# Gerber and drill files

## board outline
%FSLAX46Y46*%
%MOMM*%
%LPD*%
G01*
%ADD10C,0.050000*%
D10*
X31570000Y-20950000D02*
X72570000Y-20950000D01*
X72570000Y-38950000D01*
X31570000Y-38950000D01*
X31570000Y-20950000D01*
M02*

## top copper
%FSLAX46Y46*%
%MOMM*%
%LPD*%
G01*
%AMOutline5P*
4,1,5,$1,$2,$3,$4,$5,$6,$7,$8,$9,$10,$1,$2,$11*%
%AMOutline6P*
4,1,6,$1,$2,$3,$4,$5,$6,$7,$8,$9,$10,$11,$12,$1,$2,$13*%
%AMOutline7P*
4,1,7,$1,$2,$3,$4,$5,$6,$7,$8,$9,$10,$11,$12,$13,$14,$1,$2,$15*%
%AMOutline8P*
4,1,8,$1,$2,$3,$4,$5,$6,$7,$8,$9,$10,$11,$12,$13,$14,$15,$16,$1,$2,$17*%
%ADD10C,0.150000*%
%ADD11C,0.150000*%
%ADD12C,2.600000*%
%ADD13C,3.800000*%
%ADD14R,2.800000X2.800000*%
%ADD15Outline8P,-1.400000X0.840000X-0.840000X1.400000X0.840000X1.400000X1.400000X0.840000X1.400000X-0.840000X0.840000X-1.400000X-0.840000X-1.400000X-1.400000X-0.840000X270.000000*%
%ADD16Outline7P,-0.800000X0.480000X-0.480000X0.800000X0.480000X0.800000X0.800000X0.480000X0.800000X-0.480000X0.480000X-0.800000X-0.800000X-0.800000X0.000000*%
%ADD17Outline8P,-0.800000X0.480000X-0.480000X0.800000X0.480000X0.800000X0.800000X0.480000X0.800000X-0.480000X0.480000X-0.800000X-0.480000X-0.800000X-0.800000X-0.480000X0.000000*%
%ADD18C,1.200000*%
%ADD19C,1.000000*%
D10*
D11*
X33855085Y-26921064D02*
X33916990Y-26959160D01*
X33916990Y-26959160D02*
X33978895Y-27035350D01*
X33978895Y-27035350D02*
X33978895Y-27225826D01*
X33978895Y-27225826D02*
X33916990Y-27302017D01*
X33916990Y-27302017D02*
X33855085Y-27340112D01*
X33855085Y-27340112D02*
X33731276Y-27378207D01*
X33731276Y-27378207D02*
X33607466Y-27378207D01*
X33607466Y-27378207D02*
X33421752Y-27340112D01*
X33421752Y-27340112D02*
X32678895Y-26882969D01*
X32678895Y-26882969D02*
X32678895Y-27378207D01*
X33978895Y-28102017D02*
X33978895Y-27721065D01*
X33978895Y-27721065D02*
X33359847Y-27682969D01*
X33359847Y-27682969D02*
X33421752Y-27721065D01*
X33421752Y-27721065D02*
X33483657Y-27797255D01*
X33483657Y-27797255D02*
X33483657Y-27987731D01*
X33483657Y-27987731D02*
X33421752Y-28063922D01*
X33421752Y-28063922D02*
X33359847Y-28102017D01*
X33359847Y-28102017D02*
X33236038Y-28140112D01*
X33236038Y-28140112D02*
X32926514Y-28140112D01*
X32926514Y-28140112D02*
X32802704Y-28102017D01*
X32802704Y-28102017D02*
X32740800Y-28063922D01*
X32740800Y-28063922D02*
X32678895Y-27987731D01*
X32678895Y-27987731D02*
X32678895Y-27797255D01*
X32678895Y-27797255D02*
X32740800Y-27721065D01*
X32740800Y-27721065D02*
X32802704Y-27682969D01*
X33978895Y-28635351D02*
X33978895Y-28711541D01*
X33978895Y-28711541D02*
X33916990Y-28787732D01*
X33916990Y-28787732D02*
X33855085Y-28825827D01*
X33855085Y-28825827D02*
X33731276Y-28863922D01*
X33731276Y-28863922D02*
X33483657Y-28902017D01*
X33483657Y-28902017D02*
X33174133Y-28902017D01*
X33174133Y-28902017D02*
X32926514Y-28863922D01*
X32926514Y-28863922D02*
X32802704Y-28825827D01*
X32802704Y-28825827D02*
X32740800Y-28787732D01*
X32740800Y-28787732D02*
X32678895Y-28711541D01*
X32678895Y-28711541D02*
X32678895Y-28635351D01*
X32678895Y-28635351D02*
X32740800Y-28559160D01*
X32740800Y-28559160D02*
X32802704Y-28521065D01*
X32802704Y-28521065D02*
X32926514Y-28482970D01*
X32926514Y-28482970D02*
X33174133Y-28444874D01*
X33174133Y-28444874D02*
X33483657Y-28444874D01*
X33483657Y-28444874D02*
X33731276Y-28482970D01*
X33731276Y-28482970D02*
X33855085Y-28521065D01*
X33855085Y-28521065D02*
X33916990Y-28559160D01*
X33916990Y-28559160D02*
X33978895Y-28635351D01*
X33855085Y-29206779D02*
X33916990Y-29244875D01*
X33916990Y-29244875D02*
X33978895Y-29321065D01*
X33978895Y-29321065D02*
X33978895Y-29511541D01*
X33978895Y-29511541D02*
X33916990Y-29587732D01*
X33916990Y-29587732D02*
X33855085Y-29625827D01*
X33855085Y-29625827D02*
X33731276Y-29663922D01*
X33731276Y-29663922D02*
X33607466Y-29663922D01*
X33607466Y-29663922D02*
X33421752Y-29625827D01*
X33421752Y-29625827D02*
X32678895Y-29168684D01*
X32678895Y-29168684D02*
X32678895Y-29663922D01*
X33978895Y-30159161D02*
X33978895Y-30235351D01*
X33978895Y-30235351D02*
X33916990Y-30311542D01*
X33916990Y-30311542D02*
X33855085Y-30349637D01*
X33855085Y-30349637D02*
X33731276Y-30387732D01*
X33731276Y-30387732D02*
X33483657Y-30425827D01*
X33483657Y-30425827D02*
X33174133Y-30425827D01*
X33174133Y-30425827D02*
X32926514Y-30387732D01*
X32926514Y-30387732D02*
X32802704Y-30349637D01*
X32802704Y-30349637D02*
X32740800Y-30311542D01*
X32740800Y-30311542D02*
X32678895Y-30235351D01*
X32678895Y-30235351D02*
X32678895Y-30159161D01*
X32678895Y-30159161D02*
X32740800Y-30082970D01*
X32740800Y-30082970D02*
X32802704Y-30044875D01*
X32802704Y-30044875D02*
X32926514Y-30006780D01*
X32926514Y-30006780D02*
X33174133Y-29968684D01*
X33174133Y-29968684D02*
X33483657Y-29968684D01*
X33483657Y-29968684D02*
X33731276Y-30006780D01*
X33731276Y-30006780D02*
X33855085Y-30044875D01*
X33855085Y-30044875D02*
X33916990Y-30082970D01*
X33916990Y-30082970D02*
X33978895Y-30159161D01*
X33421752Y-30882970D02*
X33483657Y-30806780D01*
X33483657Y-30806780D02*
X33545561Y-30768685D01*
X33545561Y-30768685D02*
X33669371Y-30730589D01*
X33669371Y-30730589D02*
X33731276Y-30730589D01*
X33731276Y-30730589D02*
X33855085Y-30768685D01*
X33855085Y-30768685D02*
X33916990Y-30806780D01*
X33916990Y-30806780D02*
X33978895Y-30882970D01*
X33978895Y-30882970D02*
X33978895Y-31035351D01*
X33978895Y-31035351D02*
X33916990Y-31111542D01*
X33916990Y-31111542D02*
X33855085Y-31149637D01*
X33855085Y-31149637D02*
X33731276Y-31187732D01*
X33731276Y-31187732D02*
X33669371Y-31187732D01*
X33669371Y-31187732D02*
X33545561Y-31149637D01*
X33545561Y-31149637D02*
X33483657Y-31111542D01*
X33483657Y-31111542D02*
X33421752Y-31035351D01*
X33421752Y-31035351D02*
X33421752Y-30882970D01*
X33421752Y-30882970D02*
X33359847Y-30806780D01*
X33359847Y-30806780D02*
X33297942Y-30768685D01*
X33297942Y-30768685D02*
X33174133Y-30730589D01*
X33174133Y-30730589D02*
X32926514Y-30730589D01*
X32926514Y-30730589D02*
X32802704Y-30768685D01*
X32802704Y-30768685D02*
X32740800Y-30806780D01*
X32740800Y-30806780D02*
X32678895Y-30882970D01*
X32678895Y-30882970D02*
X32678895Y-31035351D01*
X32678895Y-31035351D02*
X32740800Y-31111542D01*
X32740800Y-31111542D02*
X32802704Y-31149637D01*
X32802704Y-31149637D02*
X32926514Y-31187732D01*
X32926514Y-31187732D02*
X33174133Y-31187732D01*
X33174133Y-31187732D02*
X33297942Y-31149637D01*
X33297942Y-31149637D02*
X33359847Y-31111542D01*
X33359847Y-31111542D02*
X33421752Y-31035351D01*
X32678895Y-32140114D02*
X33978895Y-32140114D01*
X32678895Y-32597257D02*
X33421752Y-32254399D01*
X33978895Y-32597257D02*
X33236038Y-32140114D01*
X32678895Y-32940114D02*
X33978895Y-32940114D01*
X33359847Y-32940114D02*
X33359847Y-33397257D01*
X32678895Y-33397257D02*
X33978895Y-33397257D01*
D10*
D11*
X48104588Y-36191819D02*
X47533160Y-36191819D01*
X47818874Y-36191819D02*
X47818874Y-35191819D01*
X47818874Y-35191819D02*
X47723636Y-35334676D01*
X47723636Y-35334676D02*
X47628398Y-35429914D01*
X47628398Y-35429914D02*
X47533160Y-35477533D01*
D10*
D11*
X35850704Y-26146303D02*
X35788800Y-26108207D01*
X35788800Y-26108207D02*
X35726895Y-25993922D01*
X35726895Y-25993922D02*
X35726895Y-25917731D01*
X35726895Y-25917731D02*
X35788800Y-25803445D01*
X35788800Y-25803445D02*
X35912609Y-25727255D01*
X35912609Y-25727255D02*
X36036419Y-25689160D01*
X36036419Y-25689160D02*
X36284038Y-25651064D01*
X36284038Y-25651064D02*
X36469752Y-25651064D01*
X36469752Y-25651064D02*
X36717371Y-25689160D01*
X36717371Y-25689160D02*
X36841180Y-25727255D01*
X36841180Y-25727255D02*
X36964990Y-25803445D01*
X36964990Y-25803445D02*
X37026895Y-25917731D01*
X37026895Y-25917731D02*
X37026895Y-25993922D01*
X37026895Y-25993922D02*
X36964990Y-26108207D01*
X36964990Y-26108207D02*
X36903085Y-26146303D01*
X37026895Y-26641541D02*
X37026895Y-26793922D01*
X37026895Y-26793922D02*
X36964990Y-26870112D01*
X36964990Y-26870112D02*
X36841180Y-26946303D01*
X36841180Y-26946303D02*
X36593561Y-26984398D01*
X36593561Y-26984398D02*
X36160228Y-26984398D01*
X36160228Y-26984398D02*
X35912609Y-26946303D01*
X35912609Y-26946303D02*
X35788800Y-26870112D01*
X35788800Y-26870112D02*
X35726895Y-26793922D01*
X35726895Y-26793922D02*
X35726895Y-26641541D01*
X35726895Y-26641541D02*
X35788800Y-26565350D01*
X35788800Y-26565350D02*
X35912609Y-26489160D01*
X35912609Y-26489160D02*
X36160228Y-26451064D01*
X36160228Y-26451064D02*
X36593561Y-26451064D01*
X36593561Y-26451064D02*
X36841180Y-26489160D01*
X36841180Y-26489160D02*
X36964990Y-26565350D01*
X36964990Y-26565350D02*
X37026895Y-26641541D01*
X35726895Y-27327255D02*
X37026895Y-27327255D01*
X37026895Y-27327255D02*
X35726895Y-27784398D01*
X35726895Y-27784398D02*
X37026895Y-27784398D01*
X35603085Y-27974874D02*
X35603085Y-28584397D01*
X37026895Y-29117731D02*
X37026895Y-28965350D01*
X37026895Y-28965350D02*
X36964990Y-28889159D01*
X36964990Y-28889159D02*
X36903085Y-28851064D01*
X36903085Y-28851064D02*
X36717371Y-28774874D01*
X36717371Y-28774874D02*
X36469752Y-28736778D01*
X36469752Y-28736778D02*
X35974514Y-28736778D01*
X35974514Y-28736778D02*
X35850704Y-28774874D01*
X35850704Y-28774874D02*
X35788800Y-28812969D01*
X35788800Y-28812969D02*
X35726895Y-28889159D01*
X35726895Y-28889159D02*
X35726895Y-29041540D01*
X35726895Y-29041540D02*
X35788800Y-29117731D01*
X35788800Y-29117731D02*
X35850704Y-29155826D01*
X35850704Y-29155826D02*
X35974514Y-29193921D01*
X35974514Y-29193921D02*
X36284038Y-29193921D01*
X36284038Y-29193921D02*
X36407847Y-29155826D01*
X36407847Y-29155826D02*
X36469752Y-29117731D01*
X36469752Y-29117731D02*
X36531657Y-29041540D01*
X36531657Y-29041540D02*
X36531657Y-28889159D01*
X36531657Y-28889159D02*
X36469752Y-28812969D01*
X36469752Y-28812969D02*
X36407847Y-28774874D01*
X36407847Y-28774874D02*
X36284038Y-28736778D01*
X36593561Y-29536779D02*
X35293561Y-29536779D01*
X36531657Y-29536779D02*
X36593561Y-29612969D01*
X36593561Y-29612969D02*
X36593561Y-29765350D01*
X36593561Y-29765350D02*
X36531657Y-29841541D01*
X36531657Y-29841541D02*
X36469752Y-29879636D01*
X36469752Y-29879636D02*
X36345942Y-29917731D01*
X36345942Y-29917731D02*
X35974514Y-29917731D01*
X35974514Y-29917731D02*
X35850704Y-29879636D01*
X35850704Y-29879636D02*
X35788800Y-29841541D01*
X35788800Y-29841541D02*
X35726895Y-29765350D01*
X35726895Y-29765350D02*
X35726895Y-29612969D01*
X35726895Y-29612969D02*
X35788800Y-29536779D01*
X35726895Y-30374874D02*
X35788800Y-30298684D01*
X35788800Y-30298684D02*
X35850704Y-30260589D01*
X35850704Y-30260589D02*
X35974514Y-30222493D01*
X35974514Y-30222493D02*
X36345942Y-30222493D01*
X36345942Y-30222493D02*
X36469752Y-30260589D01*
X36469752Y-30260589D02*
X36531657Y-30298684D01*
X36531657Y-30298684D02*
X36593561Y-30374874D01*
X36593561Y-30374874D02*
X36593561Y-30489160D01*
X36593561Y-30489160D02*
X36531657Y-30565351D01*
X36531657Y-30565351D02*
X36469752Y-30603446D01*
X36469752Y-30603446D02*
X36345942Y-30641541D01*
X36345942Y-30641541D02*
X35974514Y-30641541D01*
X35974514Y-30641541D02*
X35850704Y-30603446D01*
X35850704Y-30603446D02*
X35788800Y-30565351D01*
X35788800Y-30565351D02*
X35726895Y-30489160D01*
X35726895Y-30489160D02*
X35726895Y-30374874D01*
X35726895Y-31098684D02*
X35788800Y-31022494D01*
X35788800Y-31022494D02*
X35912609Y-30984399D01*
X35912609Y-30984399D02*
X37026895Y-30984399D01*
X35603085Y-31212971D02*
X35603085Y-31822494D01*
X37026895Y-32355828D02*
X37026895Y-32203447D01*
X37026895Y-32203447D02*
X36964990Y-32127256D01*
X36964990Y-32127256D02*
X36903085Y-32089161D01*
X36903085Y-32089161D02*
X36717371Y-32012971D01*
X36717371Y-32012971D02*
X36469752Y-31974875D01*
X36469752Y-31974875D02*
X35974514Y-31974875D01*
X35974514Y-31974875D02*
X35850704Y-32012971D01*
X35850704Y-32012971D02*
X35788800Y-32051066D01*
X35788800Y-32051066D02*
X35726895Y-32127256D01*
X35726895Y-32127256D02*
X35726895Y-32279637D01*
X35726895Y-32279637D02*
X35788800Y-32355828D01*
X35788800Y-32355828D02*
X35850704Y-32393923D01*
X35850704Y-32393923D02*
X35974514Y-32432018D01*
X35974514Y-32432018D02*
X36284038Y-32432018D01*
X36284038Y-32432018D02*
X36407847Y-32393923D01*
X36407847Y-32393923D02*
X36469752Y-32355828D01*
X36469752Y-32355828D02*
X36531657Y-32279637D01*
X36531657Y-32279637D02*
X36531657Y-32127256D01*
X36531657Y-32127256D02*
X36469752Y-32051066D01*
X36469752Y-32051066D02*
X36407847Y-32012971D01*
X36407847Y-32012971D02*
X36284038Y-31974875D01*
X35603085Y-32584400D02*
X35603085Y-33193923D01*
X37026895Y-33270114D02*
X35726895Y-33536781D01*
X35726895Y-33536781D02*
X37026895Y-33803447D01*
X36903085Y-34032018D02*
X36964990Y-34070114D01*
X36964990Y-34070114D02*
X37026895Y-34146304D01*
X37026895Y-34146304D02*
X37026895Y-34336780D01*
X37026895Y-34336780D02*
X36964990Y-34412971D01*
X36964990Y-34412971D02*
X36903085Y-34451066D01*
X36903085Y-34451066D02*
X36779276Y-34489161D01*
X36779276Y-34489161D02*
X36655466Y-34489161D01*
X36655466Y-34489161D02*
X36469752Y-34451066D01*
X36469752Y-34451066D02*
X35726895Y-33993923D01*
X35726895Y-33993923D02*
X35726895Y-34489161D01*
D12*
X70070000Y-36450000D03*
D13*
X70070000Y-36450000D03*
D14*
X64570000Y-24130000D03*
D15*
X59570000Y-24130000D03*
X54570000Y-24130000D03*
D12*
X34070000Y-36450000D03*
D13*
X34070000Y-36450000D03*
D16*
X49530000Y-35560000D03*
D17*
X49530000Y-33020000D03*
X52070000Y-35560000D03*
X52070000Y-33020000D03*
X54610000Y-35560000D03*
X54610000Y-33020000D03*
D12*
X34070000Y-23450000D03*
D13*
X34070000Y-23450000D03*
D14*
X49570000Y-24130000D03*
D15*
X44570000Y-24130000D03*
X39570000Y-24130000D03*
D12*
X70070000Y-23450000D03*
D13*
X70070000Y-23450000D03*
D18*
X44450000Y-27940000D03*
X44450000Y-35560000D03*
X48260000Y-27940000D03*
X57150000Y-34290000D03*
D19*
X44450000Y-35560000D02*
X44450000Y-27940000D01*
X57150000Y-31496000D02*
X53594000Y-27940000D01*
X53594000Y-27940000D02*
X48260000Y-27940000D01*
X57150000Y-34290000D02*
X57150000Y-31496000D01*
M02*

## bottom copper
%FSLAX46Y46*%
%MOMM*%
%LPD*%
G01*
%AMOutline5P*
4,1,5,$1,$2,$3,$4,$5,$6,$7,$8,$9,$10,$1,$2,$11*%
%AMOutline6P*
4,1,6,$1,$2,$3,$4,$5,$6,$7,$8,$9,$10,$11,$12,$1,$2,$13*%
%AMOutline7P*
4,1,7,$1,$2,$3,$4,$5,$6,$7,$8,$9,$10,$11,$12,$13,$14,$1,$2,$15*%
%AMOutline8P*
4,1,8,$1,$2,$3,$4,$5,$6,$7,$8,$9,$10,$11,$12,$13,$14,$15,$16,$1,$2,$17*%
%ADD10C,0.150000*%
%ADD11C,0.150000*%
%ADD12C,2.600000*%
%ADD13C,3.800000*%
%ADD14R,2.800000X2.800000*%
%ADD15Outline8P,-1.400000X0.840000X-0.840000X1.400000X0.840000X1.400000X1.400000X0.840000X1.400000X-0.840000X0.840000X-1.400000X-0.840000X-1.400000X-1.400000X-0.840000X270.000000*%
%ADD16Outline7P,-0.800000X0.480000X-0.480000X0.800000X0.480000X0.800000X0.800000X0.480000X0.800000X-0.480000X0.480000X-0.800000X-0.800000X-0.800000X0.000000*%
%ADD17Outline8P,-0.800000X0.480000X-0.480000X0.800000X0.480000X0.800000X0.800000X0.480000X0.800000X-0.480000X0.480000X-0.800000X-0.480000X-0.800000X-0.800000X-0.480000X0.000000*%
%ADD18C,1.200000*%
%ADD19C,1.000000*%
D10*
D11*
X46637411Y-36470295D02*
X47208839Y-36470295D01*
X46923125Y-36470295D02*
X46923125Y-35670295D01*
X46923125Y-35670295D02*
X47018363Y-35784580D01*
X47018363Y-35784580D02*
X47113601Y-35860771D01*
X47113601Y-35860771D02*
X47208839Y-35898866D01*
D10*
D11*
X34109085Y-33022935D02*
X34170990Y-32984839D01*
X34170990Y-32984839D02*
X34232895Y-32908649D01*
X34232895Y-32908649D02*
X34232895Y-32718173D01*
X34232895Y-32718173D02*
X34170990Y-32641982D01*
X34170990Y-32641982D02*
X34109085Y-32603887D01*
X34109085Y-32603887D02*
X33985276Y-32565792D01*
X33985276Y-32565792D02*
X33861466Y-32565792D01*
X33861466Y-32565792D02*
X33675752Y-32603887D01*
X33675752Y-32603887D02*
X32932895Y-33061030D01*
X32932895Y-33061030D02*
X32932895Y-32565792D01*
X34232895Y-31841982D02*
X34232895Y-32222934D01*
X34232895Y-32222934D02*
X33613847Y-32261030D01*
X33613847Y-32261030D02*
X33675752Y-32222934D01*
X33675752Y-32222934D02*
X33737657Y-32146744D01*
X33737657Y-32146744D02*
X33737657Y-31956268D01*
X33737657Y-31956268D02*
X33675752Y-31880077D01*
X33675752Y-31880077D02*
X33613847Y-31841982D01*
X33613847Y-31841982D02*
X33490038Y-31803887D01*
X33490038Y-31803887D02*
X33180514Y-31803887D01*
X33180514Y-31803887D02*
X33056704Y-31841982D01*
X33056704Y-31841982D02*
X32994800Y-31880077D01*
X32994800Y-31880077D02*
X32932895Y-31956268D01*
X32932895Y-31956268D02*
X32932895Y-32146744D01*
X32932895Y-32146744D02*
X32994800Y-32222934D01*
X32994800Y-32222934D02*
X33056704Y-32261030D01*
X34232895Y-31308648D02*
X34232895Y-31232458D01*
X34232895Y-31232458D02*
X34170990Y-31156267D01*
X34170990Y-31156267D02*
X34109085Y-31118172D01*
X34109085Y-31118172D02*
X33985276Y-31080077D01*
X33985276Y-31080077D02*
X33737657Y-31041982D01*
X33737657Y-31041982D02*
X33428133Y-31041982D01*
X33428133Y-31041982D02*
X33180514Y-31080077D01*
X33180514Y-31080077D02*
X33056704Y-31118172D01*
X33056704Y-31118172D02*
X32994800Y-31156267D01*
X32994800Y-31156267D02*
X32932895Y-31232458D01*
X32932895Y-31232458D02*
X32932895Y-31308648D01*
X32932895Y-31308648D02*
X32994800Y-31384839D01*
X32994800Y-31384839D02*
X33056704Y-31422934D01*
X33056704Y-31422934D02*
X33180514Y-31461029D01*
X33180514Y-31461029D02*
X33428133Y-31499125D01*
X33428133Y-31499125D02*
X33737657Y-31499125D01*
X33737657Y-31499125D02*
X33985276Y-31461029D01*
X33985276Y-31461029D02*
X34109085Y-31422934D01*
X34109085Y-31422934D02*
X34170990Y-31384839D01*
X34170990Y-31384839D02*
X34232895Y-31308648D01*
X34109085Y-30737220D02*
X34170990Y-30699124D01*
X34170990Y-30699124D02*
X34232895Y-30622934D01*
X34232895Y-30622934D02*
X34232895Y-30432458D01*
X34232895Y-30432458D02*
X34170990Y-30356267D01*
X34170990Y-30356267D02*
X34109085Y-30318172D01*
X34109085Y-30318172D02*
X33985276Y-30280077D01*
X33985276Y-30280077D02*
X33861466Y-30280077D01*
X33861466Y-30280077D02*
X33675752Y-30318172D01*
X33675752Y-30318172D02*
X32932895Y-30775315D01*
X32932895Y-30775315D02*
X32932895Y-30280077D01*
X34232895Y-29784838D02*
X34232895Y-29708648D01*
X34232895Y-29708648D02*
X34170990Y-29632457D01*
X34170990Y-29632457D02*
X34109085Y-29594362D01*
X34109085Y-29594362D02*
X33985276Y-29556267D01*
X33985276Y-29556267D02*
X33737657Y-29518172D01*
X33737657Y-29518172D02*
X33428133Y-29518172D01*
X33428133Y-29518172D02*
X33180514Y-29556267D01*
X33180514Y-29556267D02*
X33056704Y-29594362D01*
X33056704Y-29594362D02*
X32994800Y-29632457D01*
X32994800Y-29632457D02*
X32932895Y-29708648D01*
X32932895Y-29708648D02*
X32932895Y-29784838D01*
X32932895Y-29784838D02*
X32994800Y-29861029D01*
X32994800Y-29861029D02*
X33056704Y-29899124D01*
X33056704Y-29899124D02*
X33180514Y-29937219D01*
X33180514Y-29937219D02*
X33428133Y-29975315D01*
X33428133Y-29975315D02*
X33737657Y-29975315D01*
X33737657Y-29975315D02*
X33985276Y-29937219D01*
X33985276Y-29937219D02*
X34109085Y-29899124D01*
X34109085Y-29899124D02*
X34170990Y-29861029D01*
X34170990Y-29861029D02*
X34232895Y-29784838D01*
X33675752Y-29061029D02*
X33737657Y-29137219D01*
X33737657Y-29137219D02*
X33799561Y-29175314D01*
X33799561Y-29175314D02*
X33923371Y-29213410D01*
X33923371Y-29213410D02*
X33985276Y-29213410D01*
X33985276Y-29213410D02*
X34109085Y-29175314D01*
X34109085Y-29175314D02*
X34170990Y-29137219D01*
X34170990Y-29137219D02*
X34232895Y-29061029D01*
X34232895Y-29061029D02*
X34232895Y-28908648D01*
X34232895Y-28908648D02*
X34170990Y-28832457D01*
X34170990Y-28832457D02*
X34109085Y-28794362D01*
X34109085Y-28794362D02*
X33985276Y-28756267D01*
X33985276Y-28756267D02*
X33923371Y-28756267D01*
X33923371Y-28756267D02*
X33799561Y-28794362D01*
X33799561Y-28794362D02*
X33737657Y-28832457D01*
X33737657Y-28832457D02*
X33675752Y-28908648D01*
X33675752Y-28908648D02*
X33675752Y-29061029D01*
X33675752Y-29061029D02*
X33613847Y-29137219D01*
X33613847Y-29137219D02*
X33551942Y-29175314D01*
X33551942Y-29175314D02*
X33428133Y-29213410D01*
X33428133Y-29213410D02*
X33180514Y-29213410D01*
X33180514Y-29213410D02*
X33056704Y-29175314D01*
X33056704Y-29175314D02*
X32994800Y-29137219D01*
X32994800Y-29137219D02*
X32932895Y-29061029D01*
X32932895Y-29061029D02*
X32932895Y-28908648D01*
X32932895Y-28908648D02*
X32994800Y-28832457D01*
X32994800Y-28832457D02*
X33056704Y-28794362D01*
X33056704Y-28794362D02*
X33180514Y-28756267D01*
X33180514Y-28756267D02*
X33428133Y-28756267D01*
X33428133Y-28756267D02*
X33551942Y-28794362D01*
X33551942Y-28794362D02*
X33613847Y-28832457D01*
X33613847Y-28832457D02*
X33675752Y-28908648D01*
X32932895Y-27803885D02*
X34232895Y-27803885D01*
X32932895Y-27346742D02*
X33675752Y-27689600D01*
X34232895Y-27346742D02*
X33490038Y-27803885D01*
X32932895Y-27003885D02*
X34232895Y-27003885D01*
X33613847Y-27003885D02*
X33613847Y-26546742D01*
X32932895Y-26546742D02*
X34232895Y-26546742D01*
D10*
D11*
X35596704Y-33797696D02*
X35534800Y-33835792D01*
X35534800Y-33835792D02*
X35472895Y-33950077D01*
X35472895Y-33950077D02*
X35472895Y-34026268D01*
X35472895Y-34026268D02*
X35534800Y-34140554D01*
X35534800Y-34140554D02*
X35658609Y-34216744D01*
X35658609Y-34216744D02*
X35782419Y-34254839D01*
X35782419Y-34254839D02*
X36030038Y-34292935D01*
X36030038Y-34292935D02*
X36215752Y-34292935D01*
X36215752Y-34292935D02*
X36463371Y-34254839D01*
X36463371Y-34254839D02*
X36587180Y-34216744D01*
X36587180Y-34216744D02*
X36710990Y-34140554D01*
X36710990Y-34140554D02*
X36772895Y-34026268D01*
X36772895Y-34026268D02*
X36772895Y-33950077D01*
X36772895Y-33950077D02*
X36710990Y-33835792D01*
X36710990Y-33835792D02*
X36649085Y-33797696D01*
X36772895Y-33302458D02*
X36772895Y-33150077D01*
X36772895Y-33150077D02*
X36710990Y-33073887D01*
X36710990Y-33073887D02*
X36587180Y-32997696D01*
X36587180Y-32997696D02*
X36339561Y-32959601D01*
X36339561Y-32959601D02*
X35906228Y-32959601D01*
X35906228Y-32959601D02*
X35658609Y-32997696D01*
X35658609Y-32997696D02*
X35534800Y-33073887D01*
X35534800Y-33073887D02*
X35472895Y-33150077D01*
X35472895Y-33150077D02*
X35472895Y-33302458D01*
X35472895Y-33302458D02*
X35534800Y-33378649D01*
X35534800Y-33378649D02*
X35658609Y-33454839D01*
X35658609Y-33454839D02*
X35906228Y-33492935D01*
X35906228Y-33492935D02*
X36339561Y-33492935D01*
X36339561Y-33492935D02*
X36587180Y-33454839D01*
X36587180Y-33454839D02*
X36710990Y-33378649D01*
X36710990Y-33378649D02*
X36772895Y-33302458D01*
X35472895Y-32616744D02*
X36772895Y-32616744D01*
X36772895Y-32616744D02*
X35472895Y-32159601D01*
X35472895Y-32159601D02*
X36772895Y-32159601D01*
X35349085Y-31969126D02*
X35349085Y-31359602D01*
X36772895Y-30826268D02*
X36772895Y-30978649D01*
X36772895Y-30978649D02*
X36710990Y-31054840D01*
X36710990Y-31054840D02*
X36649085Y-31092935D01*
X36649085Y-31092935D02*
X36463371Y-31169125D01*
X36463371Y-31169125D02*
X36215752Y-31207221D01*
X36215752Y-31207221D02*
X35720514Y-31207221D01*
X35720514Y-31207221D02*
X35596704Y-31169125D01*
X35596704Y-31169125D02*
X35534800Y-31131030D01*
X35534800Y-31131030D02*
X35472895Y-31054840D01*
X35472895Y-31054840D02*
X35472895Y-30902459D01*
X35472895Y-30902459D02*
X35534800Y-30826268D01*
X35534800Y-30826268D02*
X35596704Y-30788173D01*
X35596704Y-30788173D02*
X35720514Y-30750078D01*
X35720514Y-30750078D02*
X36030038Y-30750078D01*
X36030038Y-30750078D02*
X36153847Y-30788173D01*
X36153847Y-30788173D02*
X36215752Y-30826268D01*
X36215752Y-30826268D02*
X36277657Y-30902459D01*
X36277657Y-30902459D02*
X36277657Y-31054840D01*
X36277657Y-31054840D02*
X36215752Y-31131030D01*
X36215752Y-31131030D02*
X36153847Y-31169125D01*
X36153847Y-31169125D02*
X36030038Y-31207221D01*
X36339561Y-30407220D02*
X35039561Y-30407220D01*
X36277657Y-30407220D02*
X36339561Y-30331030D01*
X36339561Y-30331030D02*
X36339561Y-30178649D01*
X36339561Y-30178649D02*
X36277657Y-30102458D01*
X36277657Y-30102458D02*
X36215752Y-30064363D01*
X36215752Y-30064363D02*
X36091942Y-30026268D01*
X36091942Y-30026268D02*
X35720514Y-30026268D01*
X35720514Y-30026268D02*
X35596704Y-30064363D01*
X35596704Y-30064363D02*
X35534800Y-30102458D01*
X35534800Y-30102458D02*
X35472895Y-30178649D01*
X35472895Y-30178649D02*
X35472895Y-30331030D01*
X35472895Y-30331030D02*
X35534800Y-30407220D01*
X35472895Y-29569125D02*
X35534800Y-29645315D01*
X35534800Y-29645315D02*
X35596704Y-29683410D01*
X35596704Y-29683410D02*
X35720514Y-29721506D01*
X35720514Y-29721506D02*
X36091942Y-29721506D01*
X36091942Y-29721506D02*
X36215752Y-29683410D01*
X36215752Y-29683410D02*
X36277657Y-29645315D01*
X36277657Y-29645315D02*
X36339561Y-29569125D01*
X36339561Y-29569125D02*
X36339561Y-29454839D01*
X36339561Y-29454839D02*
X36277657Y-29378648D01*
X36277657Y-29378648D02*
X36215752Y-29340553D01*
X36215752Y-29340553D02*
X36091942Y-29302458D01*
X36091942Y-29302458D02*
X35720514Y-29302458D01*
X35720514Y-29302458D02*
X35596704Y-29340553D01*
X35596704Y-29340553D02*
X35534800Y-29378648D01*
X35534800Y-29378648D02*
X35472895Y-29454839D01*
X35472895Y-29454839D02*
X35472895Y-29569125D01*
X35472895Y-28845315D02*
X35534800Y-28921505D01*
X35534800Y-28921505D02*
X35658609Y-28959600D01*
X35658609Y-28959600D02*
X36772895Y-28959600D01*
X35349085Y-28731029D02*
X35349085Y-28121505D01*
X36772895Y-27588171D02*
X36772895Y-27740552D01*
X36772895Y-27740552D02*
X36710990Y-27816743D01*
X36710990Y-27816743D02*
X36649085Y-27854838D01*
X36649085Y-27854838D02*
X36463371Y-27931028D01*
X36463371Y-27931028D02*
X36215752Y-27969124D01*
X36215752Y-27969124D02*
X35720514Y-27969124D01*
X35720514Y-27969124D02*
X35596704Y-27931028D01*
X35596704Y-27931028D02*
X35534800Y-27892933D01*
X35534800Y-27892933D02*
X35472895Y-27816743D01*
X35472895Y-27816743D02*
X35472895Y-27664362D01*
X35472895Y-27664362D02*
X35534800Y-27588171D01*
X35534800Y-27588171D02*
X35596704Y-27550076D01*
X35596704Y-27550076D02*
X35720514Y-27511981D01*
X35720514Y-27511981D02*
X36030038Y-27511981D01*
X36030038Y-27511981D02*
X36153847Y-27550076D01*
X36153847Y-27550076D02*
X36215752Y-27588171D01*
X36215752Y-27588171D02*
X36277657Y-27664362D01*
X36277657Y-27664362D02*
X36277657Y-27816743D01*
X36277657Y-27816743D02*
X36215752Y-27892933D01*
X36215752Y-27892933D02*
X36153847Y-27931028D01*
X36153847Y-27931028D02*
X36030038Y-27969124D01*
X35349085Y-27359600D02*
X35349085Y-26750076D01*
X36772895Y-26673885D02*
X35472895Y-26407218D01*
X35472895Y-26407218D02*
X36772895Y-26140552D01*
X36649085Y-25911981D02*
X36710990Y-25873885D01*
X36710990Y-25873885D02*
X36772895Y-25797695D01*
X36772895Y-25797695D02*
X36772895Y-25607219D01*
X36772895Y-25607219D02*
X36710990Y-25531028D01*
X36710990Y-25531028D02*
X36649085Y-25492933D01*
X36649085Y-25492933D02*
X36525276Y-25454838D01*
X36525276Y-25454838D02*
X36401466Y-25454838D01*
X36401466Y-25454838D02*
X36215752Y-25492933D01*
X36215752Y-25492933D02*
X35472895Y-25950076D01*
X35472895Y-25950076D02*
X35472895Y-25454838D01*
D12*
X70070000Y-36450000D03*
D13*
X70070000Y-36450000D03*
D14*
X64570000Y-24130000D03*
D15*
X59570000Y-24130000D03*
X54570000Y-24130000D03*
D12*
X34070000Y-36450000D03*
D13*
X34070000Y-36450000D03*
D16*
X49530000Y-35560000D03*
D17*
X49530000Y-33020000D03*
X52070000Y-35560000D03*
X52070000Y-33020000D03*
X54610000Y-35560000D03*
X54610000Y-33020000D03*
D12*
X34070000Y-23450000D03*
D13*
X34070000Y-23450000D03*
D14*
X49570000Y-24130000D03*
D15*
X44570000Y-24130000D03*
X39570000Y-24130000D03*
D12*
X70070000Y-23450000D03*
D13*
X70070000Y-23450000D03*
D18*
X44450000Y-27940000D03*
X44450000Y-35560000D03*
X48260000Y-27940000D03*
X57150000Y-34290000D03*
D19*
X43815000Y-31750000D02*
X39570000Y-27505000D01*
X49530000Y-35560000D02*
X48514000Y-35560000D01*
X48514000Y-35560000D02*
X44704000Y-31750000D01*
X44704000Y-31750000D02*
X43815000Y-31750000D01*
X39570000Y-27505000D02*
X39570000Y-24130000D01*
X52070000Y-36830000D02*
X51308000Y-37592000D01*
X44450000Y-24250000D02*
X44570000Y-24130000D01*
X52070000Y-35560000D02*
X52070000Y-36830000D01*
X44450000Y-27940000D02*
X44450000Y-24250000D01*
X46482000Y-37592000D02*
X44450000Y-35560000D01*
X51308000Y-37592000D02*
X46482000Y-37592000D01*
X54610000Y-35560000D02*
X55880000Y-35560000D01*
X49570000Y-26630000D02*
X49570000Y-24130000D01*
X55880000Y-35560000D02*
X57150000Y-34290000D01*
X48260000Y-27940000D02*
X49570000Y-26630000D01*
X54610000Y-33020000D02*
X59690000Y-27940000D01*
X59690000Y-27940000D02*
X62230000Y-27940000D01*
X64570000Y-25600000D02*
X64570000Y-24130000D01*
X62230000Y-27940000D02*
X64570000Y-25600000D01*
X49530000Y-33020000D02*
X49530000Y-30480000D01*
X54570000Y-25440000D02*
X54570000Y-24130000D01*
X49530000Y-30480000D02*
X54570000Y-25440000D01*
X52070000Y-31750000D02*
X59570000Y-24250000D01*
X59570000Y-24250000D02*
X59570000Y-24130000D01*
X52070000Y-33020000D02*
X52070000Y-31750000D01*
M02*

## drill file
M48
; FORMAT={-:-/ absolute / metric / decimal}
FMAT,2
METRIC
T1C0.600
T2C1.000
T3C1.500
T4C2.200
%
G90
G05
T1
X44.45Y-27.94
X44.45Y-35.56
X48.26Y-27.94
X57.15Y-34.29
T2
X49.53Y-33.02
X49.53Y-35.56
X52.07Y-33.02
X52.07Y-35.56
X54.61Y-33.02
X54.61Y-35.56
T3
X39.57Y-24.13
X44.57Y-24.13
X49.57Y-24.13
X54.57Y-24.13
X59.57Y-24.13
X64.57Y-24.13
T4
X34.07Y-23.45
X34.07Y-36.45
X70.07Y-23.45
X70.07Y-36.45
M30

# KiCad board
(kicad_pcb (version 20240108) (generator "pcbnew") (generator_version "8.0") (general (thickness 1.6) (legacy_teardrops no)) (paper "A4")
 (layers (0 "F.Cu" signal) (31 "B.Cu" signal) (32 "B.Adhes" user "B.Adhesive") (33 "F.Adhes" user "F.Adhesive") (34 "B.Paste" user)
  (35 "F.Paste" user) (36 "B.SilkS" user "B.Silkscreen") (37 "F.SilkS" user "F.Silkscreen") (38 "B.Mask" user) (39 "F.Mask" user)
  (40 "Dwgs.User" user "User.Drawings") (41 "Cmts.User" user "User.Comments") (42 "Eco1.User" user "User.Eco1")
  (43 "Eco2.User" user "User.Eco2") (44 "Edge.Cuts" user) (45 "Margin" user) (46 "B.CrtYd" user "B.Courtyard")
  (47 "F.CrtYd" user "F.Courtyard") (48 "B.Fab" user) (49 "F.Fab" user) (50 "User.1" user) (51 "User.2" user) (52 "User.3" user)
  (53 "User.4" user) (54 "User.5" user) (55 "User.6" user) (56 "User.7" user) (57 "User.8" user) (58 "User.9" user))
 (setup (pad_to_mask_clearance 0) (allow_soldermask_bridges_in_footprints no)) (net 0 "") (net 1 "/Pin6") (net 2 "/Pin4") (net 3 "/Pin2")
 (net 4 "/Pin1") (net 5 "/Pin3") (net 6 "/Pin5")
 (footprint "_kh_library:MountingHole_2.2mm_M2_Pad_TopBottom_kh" (layer "F.Cu") (at 70.07 36.45)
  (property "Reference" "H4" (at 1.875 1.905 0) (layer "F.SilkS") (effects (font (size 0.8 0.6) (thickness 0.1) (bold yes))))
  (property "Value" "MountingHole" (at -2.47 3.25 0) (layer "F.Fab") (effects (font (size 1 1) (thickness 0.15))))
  (pad "1" thru_hole circle (at 0 0) (size 2.6 2.6) (drill 2.2) (layers "*.Cu" "*.Mask") (remove_unused_layers no))
  (pad "1" connect circle (at 0 0) (size 3.8 3.8) (layers "F.Cu" "F.Mask"))
  (pad "1" connect circle (at 0 0) (size 3.8 3.8) (layers "B.Cu" "B.Mask")))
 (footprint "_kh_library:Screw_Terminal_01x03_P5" (layer "F.Cu") (at 64.57 24.13 -90)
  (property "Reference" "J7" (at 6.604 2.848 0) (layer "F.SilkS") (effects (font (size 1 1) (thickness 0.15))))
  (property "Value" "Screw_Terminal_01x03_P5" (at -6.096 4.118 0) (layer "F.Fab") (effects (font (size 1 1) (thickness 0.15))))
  (pad "1" thru_hole rect (at 0 0 270) (size 2.8 2.8) (drill 1.5) (layers "*.Cu" "*.Mask") (remove_unused_layers no) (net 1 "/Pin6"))
  (pad "2" thru_hole roundrect (at 0 5 270) (size 2.8 2.8) (drill 1.5) (layers "*.Cu" "*.Mask") (remove_unused_layers no)
   (roundrect_rratio 0) (chamfer_ratio 0.2) (chamfer top_left top_right bottom_left bottom_right) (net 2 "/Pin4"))
  (pad "3" thru_hole roundrect (at 0 10 270) (size 2.8 2.8) (drill 1.5) (layers "*.Cu" "*.Mask") (remove_unused_layers no)
   (roundrect_rratio 0) (chamfer_ratio 0.2) (chamfer top_left top_right bottom_left bottom_right) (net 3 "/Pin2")))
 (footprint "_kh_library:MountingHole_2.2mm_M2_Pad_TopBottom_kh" (layer "F.Cu") (at 34.07 36.45)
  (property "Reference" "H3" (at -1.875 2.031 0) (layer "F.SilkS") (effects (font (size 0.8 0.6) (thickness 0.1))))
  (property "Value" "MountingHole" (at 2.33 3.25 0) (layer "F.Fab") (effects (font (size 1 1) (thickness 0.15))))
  (pad "1" thru_hole circle (at 0 0) (size 2.6 2.6) (drill 2.2) (layers "*.Cu" "*.Mask") (remove_unused_layers no))
  (pad "1" connect circle (at 0 0) (size 3.8 3.8) (layers "F.Cu" "F.Mask"))
  (pad "1" connect circle (at 0 0) (size 3.8 3.8) (layers "B.Cu" "B.Mask")))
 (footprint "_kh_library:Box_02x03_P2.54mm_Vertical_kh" (layer "F.Cu") (at 49.53 35.56)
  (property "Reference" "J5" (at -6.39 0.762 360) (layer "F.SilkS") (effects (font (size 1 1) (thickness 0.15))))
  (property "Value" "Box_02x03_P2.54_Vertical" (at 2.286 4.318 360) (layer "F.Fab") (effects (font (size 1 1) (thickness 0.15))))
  (pad "1" thru_hole roundrect (at 0 0) (size 1.6 1.6) (drill 1) (layers "*.Cu" "*.Mask") (remove_unused_layers no) (roundrect_rratio 0)
   (chamfer_ratio 0.2) (chamfer top_left top_right bottom_right) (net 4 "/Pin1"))
  (pad "2" thru_hole roundrect (at 0 -2.54) (size 1.6 1.6) (drill 1) (layers "*.Cu" "*.Mask") (remove_unused_layers no) (roundrect_rratio 0)
   (chamfer_ratio 0.2) (chamfer top_left top_right bottom_left bottom_right) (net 3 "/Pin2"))
  (pad "3" thru_hole roundrect (at 2.54 0) (size 1.6 1.6) (drill 1) (layers "*.Cu" "*.Mask") (remove_unused_layers no) (roundrect_rratio 0)
   (chamfer_ratio 0.2) (chamfer top_left top_right bottom_left bottom_right) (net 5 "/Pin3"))
  (pad "4" thru_hole roundrect (at 2.54 -2.54) (size 1.6 1.6) (drill 1) (layers "*.Cu" "*.Mask") (remove_unused_layers no)
   (roundrect_rratio 0) (chamfer_ratio 0.2) (chamfer top_left top_right bottom_left bottom_right) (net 2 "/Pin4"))
  (pad "5" thru_hole roundrect (at 5.08 0) (size 1.6 1.6) (drill 1) (layers "*.Cu" "*.Mask") (remove_unused_layers no) (roundrect_rratio 0)
   (chamfer_ratio 0.2) (chamfer top_left top_right bottom_left bottom_right) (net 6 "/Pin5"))
  (pad "6" thru_hole roundrect (at 5.08 -2.54) (size 1.6 1.6) (drill 1) (layers "*.Cu" "*.Mask") (remove_unused_layers no)
   (roundrect_rratio 0) (chamfer_ratio 0.2) (chamfer top_left top_right bottom_left bottom_right) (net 1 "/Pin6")))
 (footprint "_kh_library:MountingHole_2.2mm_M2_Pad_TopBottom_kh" (layer "F.Cu") (at 34.07 23.45)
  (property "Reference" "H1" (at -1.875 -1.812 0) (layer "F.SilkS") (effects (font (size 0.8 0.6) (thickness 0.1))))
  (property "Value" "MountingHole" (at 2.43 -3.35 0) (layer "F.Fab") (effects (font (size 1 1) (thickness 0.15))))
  (pad "1" thru_hole circle (at 0 0) (size 2.6 2.6) (drill 2.2) (layers "*.Cu" "*.Mask") (remove_unused_layers no))
  (pad "1" connect circle (at 0 0) (size 3.8 3.8) (layers "F.Cu" "F.Mask"))
  (pad "1" connect circle (at 0 0) (size 3.8 3.8) (layers "B.Cu" "B.Mask")))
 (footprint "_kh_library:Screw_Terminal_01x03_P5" (layer "F.Cu") (at 49.57 24.13 -90)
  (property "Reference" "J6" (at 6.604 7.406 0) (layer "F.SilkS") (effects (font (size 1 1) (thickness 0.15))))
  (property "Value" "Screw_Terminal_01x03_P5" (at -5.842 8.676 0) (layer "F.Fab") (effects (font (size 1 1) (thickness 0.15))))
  (pad "1" thru_hole rect (at 0 0 270) (size 2.8 2.8) (drill 1.5) (layers "*.Cu" "*.Mask") (remove_unused_layers no) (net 6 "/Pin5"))
  (pad "2" thru_hole roundrect (at 0 5 270) (size 2.8 2.8) (drill 1.5) (layers "*.Cu" "*.Mask") (remove_unused_layers no)
   (roundrect_rratio 0) (chamfer_ratio 0.2) (chamfer top_left top_right bottom_left bottom_right) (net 5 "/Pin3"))
  (pad "3" thru_hole roundrect (at 0 10 270) (size 2.8 2.8) (drill 1.5) (layers "*.Cu" "*.Mask") (remove_unused_layers no)
   (roundrect_rratio 0) (chamfer_ratio 0.2) (chamfer top_left top_right bottom_left bottom_right) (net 4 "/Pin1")))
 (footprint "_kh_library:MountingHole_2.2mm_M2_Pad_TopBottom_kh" (layer "F.Cu") (at 70.07 23.45)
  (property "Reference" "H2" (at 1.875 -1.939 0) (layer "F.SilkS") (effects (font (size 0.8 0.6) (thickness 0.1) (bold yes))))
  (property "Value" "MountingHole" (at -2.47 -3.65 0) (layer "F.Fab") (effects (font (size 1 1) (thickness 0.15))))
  (pad "1" thru_hole circle (at 0 0) (size 2.6 2.6) (drill 2.2) (layers "*.Cu" "*.Mask") (remove_unused_layers no))
  (pad "1" connect circle (at 0 0) (size 3.8 3.8) (layers "F.Cu" "F.Mask"))
  (pad "1" connect circle (at 0 0) (size 3.8 3.8) (layers "B.Cu" "B.Mask")))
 (gr_rect (start 31.57 20.95) (end 72.57 38.95) (stroke (width 0.05) (type default)) (fill none) (layer "Edge.Cuts"))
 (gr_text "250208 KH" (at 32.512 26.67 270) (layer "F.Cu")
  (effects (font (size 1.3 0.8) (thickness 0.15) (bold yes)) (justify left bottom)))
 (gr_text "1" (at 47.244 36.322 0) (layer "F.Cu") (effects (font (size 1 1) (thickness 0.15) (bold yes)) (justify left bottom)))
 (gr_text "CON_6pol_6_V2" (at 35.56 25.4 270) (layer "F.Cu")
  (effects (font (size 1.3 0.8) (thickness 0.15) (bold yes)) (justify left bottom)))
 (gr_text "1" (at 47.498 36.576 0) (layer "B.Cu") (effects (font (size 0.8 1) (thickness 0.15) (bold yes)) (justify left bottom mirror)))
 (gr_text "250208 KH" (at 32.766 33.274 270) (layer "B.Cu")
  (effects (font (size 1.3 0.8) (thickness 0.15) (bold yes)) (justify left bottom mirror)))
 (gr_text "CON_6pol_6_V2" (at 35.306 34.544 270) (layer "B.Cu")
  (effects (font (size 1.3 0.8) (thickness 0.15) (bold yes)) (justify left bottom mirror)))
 (segment (start 43.815 31.75) (end 39.57 27.505) (width 1) (layer "B.Cu") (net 4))
 (segment (start 49.53 35.56) (end 48.514 35.56) (width 1) (layer "B.Cu") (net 4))
 (segment (start 48.514 35.56) (end 44.704 31.75) (width 1) (layer "B.Cu") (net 4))
 (segment (start 44.704 31.75) (end 43.815 31.75) (width 1) (layer "B.Cu") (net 4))
 (segment (start 39.57 27.505) (end 39.57 24.13) (width 1) (layer "B.Cu") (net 4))
 (segment (start 44.45 35.56) (end 44.45 27.94) (width 1) (layer "F.Cu") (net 5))
 (via (at 44.45 27.94) (size 1.2) (drill 0.6) (layers "F.Cu" "B.Cu") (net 5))
 (via (at 44.45 35.56) (size 1.2) (drill 0.6) (layers "F.Cu" "B.Cu") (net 5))
 (segment (start 52.07 36.83) (end 51.308 37.592) (width 1) (layer "B.Cu") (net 5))
 (segment (start 44.45 24.25) (end 44.57 24.13) (width 1) (layer "B.Cu") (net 5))
 (segment (start 52.07 35.56) (end 52.07 36.83) (width 1) (layer "B.Cu") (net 5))
 (segment (start 44.45 27.94) (end 44.45 24.25) (width 1) (layer "B.Cu") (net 5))
 (segment (start 46.482 37.592) (end 44.45 35.56) (width 1) (layer "B.Cu") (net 5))
 (segment (start 51.308 37.592) (end 46.482 37.592) (width 1) (layer "B.Cu") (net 5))
 (segment (start 57.15 31.496) (end 53.594 27.94) (width 1) (layer "F.Cu") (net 6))
 (segment (start 53.594 27.94) (end 48.26 27.94) (width 1) (layer "F.Cu") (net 6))
 (segment (start 57.15 34.29) (end 57.15 31.496) (width 1) (layer "F.Cu") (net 6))
 (via (at 48.26 27.94) (size 1.2) (drill 0.6) (layers "F.Cu" "B.Cu") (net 6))
 (via (at 57.15 34.29) (size 1.2) (drill 0.6) (layers "F.Cu" "B.Cu") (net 6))
 (segment (start 54.61 35.56) (end 55.88 35.56) (width 1) (layer "B.Cu") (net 6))
 (segment (start 49.57 26.63) (end 49.57 24.13) (width 1) (layer "B.Cu") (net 6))
 (segment (start 55.88 35.56) (end 57.15 34.29) (width 1) (layer "B.Cu") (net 6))
 (segment (start 48.26 27.94) (end 49.57 26.63) (width 1) (layer "B.Cu") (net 6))
 (segment (start 54.61 33.02) (end 59.69 27.94) (width 1) (layer "B.Cu") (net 1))
 (segment (start 59.69 27.94) (end 62.23 27.94) (width 1) (layer "B.Cu") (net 1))
 (segment (start 64.57 25.6) (end 64.57 24.13) (width 1) (layer "B.Cu") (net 1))
 (segment (start 62.23 27.94) (end 64.57 25.6) (width 1) (layer "B.Cu") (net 1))
 (segment (start 49.53 33.02) (end 49.53 30.48) (width 1) (layer "B.Cu") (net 3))
 (segment (start 54.57 25.44) (end 54.57 24.13) (width 1) (layer "B.Cu") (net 3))
 (segment (start 49.53 30.48) (end 54.57 25.44) (width 1) (layer "B.Cu") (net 3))
 (segment (start 52.07 31.75) (end 59.57 24.25) (width 1) (layer "B.Cu") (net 2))
 (segment (start 59.57 24.25) (end 59.57 24.13) (width 1) (layer "B.Cu") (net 2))
 (segment (start 52.07 33.02) (end 52.07 31.75) (width 1) (layer "B.Cu") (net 2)))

